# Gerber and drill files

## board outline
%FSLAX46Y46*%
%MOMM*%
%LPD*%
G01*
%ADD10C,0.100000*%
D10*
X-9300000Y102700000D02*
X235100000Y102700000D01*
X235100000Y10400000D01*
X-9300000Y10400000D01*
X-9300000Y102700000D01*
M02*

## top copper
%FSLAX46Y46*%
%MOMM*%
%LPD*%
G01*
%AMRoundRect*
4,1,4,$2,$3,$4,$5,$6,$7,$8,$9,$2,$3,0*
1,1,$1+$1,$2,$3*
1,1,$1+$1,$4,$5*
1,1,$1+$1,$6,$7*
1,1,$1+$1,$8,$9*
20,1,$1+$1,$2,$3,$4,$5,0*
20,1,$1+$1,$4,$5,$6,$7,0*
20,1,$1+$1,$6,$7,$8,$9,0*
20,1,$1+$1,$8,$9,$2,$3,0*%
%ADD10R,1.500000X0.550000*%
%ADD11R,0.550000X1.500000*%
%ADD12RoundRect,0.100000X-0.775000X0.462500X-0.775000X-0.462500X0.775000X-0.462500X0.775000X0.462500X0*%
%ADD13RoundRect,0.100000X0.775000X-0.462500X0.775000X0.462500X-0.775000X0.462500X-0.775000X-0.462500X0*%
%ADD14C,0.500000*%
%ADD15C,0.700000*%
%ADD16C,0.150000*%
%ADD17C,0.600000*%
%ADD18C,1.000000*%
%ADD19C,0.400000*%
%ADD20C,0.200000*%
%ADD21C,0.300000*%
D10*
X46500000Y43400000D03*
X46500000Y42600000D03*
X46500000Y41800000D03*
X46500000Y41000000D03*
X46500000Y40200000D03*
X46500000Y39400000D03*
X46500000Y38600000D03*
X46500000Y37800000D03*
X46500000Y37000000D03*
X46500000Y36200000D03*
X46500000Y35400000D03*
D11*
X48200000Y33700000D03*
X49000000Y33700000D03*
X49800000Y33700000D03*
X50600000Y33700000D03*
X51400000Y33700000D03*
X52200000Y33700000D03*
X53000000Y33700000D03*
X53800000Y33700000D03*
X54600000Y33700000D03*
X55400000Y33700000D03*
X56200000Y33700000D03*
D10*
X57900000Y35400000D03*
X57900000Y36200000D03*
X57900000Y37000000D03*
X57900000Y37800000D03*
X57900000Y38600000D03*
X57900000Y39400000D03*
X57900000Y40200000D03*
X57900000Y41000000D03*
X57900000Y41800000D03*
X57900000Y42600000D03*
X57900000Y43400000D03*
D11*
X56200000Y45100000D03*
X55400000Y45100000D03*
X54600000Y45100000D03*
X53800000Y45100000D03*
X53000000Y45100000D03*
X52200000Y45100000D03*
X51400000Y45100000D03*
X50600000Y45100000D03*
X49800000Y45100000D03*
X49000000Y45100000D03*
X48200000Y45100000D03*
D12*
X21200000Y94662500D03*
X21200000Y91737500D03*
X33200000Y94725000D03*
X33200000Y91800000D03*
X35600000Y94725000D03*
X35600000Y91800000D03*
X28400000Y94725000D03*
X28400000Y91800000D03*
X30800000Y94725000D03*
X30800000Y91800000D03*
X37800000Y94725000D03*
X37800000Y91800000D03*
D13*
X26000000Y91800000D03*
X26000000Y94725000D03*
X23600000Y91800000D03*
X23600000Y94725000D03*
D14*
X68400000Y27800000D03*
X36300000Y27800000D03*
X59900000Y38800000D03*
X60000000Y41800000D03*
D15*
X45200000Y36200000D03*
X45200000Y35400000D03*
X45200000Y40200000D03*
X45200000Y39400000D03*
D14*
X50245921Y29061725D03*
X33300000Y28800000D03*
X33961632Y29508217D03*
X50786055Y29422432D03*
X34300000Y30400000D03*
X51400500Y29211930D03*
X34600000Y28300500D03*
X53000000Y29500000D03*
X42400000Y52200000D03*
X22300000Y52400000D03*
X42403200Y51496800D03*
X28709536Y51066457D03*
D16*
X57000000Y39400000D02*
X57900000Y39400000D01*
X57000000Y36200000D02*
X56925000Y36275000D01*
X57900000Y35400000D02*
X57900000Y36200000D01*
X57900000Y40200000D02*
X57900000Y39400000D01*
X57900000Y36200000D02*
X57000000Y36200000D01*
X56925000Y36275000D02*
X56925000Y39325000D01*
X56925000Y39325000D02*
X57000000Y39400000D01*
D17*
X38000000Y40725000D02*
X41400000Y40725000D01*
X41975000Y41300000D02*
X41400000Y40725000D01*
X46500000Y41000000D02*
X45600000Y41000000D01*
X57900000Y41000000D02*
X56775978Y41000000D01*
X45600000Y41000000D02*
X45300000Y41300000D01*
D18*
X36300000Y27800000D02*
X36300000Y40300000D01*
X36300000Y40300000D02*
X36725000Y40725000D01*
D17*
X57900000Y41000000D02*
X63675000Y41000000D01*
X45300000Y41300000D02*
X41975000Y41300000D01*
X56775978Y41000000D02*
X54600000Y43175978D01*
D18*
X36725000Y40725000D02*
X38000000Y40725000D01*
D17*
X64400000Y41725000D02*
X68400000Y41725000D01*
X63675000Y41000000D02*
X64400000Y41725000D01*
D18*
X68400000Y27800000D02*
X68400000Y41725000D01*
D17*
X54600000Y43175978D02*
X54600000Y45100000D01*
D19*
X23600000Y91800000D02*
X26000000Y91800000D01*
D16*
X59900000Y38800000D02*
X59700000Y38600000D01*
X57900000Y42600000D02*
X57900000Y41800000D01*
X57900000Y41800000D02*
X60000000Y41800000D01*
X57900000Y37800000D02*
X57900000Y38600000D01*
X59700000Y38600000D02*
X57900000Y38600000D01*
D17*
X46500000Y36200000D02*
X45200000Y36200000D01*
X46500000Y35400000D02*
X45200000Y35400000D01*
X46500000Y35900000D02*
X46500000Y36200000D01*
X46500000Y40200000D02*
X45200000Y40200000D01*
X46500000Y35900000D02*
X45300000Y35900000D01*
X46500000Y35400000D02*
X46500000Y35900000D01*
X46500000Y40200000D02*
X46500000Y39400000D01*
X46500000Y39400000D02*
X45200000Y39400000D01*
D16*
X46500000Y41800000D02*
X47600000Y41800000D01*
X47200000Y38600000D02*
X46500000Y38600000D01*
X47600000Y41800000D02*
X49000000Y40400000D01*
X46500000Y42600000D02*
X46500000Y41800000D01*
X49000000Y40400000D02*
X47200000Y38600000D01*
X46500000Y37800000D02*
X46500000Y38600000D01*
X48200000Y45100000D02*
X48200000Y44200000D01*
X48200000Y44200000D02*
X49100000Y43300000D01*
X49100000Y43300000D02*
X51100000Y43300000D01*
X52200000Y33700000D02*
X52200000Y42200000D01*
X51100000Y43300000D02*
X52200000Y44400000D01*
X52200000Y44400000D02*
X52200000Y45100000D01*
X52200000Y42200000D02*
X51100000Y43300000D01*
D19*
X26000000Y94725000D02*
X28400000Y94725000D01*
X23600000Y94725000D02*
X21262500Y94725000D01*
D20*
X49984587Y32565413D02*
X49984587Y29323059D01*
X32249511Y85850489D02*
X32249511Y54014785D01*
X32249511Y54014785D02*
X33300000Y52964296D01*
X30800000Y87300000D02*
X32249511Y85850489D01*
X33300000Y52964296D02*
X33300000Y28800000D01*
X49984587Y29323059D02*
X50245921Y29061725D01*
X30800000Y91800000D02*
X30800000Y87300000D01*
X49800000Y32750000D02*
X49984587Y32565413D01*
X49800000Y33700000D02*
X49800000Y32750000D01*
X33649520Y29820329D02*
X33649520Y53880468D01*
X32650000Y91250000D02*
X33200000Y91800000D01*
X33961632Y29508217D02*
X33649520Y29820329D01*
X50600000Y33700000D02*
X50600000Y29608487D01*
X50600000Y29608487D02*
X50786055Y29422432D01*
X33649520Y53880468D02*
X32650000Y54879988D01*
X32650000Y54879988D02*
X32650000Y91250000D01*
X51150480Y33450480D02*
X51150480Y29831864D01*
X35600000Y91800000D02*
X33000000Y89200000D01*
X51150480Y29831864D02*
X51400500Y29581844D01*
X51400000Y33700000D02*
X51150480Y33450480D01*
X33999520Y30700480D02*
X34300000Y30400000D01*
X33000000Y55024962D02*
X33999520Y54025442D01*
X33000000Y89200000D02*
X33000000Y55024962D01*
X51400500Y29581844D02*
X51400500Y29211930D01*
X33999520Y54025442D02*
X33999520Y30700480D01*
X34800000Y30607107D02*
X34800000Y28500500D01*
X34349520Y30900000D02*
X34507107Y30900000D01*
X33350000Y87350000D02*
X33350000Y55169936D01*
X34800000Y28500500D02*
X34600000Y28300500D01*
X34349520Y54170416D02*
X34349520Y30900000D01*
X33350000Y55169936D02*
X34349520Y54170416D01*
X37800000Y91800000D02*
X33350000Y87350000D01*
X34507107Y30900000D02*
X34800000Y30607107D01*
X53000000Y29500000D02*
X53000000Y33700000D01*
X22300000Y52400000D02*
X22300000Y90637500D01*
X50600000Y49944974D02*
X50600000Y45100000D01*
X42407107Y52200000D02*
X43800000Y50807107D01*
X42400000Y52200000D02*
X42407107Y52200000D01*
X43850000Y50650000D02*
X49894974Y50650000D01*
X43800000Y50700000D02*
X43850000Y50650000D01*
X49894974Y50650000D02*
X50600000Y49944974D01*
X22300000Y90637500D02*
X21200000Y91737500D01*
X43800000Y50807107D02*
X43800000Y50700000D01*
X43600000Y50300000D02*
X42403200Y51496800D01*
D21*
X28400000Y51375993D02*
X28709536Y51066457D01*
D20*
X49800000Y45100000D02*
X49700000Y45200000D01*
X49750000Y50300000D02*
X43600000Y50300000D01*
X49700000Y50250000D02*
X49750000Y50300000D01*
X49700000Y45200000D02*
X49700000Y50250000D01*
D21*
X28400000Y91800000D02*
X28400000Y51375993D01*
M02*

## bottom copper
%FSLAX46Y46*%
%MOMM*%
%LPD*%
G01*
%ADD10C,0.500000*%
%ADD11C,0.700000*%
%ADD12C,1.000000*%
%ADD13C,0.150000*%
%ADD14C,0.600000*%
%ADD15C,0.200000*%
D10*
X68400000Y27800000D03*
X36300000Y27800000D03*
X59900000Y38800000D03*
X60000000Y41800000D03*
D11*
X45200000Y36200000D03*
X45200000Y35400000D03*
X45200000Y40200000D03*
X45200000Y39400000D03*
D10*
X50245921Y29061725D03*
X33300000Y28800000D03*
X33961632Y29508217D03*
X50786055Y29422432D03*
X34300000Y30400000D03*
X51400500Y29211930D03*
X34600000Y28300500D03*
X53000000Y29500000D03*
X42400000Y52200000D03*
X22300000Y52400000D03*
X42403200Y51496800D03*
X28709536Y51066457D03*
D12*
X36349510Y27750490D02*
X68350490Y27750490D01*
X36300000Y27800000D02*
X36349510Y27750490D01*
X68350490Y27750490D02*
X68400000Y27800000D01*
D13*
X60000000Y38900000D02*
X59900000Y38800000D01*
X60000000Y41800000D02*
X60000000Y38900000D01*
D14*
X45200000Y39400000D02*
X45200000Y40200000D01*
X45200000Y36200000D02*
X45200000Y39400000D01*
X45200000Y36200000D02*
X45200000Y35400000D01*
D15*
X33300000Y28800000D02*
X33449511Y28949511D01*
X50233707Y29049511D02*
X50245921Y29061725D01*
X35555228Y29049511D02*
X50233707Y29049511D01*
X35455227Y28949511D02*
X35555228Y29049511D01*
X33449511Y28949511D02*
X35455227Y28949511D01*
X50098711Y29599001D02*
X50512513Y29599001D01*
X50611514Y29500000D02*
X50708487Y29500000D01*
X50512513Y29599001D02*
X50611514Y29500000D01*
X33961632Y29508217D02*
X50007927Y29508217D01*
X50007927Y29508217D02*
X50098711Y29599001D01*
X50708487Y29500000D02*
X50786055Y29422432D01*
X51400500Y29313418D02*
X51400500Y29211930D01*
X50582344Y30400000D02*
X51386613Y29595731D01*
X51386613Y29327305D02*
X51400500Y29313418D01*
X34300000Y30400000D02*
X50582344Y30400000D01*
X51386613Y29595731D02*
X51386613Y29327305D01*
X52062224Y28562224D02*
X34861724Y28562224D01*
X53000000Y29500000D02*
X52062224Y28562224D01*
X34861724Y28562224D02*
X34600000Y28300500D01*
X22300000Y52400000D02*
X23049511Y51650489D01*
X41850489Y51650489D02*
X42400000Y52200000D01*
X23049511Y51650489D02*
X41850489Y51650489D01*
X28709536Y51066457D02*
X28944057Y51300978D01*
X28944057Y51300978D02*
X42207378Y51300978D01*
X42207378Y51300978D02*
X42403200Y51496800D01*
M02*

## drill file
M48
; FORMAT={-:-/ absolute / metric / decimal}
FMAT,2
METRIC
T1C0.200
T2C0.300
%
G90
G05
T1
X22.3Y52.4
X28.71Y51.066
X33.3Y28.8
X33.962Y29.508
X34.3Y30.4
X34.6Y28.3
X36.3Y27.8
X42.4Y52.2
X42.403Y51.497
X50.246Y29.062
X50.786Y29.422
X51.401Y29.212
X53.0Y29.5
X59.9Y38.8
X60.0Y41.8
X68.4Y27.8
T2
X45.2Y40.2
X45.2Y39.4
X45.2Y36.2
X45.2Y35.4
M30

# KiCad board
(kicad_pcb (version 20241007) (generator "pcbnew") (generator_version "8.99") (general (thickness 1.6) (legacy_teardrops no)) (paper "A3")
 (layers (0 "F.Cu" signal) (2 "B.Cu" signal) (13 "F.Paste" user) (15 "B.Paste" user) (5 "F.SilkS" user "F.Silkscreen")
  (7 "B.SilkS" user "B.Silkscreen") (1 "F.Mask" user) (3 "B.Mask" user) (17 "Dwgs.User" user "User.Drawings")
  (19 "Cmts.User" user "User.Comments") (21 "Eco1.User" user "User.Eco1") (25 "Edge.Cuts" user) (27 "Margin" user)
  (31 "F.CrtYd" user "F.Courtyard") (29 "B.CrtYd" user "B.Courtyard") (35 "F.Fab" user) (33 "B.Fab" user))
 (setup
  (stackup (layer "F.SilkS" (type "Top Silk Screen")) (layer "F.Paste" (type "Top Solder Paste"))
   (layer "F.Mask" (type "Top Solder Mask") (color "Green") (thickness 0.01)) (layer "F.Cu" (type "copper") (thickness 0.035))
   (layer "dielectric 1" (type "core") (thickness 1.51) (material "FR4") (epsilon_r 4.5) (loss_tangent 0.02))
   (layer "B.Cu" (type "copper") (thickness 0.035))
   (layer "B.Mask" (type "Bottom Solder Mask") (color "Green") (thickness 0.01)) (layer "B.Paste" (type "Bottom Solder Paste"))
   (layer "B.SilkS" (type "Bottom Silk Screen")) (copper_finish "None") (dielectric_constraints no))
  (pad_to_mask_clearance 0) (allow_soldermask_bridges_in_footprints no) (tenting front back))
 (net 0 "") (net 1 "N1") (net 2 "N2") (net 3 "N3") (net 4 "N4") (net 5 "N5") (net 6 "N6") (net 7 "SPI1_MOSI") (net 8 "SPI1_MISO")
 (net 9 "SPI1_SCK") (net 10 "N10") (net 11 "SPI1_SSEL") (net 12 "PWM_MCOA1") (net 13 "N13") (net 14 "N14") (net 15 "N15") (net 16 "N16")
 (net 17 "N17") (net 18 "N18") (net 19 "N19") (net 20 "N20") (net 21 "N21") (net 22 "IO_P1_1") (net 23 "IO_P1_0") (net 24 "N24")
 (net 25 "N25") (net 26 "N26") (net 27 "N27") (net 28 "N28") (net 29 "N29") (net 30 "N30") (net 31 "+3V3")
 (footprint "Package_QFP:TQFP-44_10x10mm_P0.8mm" (layer "F.Cu") (at 52.2 -39.4)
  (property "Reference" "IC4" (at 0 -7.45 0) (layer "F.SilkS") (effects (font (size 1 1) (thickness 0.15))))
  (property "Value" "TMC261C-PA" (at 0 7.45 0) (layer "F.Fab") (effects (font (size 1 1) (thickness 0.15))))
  (pad "1" smd rect (at -5.7 -4) (size 1.5 0.55) (layers "F.Cu" "F.Mask" "F.Paste"))
  (pad "2" smd rect (at -5.7 -3.2) (size 1.5 0.55) (layers "F.Cu" "F.Mask" "F.Paste") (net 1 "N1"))
  (pad "3" smd rect (at -5.7 -2.4) (size 1.5 0.55) (layers "F.Cu" "F.Mask" "F.Paste") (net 1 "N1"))
  (pad "4" smd rect (at -5.7 -1.6) (size 1.5 0.55) (layers "F.Cu" "F.Mask" "F.Paste") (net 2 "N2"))
  (pad "5" smd rect (at -5.7 -0.8) (size 1.5 0.55) (layers "F.Cu" "F.Mask" "F.Paste") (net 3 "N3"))
  (pad "6" smd rect (at -5.7 0) (size 1.5 0.55) (layers "F.Cu" "F.Mask" "F.Paste") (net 3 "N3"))
  (pad "7" smd rect (at -5.7 0.8) (size 1.5 0.55) (layers "F.Cu" "F.Mask" "F.Paste") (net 1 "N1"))
  (pad "8" smd rect (at -5.7 1.6) (size 1.5 0.55) (layers "F.Cu" "F.Mask" "F.Paste") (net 1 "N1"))
  (pad "9" smd rect (at -5.7 2.4) (size 1.5 0.55) (layers "F.Cu" "F.Mask" "F.Paste") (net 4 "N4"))
  (pad "10" smd rect (at -5.7 3.2) (size 1.5 0.55) (layers "F.Cu" "F.Mask" "F.Paste") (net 3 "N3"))
  (pad "11" smd rect (at -5.7 4) (size 1.5 0.55) (layers "F.Cu" "F.Mask" "F.Paste") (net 3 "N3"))
  (pad "12" smd rect (at -4 5.7 90) (size 1.5 0.55) (layers "F.Cu" "F.Mask" "F.Paste") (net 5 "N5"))
  (pad "13" smd rect (at -3.2 5.7 90) (size 1.5 0.55) (layers "F.Cu" "F.Mask" "F.Paste") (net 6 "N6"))
  (pad "14" smd rect (at -2.4 5.7 90) (size 1.5 0.55) (layers "F.Cu" "F.Mask" "F.Paste") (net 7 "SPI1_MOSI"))
  (pad "15" smd rect (at -1.6 5.7 90) (size 1.5 0.55) (layers "F.Cu" "F.Mask" "F.Paste") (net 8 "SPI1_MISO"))
  (pad "16" smd rect (at -0.8 5.7 90) (size 1.5 0.55) (layers "F.Cu" "F.Mask" "F.Paste") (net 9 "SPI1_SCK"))
  (pad "17" smd rect (at 0 5.7 90) (size 1.5 0.55) (layers "F.Cu" "F.Mask" "F.Paste") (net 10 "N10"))
  (pad "18" smd rect (at 0.8 5.7 90) (size 1.5 0.55) (layers "F.Cu" "F.Mask" "F.Paste") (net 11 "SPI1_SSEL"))
  (pad "19" smd rect (at 1.6 5.7 90) (size 1.5 0.55) (layers "F.Cu" "F.Mask" "F.Paste") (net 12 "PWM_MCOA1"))
  (pad "20" smd rect (at 2.4 5.7 90) (size 1.5 0.55) (layers "F.Cu" "F.Mask" "F.Paste"))
  (pad "21" smd rect (at 3.2 5.7 90) (size 1.5 0.55) (layers "F.Cu" "F.Mask" "F.Paste") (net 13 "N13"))
  (pad "22" smd rect (at 4 5.7 90) (size 1.5 0.55) (layers "F.Cu" "F.Mask" "F.Paste") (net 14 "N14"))
  (pad "23" smd rect (at 5.7 4) (size 1.5 0.55) (layers "F.Cu" "F.Mask" "F.Paste") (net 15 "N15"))
  (pad "24" smd rect (at 5.7 3.2) (size 1.5 0.55) (layers "F.Cu" "F.Mask" "F.Paste") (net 15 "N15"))
  (pad "25" smd rect (at 5.7 2.4) (size 1.5 0.55) (layers "F.Cu" "F.Mask" "F.Paste") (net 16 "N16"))
  (pad "26" smd rect (at 5.7 1.6) (size 1.5 0.55) (layers "F.Cu" "F.Mask" "F.Paste") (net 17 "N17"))
  (pad "27" smd rect (at 5.7 0.8) (size 1.5 0.55) (layers "F.Cu" "F.Mask" "F.Paste") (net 17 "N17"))
  (pad "28" smd rect (at 5.7 0) (size 1.5 0.55) (layers "F.Cu" "F.Mask" "F.Paste") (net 15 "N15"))
  (pad "29" smd rect (at 5.7 -0.8) (size 1.5 0.55) (layers "F.Cu" "F.Mask" "F.Paste") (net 15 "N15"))
  (pad "30" smd rect (at 5.7 -1.6) (size 1.5 0.55) (layers "F.Cu" "F.Mask" "F.Paste") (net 2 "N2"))
  (pad "31" smd rect (at 5.7 -2.4) (size 1.5 0.55) (layers "F.Cu" "F.Mask" "F.Paste") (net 17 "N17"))
  (pad "32" smd rect (at 5.7 -3.2) (size 1.5 0.55) (layers "F.Cu" "F.Mask" "F.Paste") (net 17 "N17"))
  (pad "33" smd rect (at 5.7 -4) (size 1.5 0.55) (layers "F.Cu" "F.Mask" "F.Paste"))
  (pad "34" smd rect (at 4 -5.7 90) (size 1.5 0.55) (layers "F.Cu" "F.Mask" "F.Paste"))
  (pad "35" smd rect (at 3.2 -5.7 90) (size 1.5 0.55) (layers "F.Cu" "F.Mask" "F.Paste") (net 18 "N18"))
  (pad "36" smd rect (at 2.4 -5.7 90) (size 1.5 0.55) (layers "F.Cu" "F.Mask" "F.Paste") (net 2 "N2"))
  (pad "37" smd rect (at 1.6 -5.7 90) (size 1.5 0.55) (layers "F.Cu" "F.Mask" "F.Paste") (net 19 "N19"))
  (pad "38" smd rect (at 0.8 -5.7 90) (size 1.5 0.55) (layers "F.Cu" "F.Mask" "F.Paste") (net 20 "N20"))
  (pad "39" smd rect (at 0 -5.7 90) (size 1.5 0.55) (layers "F.Cu" "F.Mask" "F.Paste") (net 10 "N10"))
  (pad "40" smd rect (at -0.8 -5.7 90) (size 1.5 0.55) (layers "F.Cu" "F.Mask" "F.Paste") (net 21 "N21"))
  (pad "41" smd rect (at -1.6 -5.7 90) (size 1.5 0.55) (layers "F.Cu" "F.Mask" "F.Paste") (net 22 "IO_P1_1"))
  (pad "42" smd rect (at -2.4 -5.7 90) (size 1.5 0.55) (layers "F.Cu" "F.Mask" "F.Paste") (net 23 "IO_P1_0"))
  (pad "43" smd rect (at -3.2 -5.7 90) (size 1.5 0.55) (layers "F.Cu" "F.Mask" "F.Paste") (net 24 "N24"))
  (pad "44" smd rect (at -4 -5.7 90) (size 1.5 0.55) (layers "F.Cu" "F.Mask" "F.Paste") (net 10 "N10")))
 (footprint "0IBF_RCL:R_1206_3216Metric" (layer "F.Cu") (at 21.2 -93.2 -90)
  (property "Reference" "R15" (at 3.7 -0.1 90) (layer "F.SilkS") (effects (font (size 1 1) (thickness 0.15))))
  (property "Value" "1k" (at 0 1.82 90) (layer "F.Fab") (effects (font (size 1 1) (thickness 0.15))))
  (pad "1" smd roundrect (at -1.4625 0 270) (size 1.125 1.75) (layers "F.Cu" "F.Mask" "F.Paste") (roundrect_rratio 0.08888888889)
   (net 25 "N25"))
  (pad "2" smd roundrect (at 1.4625 0 270) (size 1.125 1.75) (layers "F.Cu" "F.Mask" "F.Paste") (roundrect_rratio 0.08888888889)
   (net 22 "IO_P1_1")))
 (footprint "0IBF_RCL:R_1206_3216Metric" (layer "F.Cu") (at 33.2 -93.2625 -90)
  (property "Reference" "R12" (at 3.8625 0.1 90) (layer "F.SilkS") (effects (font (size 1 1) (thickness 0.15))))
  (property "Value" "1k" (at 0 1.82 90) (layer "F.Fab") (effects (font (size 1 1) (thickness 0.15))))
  (pad "1" smd roundrect (at -1.4625 0 270) (size 1.125 1.75) (layers "F.Cu" "F.Mask" "F.Paste") (roundrect_rratio 0.08888888889)
   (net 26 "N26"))
  (pad "2" smd roundrect (at 1.4625 0 270) (size 1.125 1.75) (layers "F.Cu" "F.Mask" "F.Paste") (roundrect_rratio 0.08888888889)
   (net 8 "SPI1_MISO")))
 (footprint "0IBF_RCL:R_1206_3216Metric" (layer "F.Cu") (at 35.6 -93.2625 -90)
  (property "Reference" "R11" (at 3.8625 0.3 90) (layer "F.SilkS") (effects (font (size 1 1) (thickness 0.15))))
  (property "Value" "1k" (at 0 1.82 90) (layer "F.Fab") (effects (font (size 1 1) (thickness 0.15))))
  (pad "1" smd roundrect (at -1.4625 0 270) (size 1.125 1.75) (layers "F.Cu" "F.Mask" "F.Paste") (roundrect_rratio 0.08888888889)
   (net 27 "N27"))
  (pad "2" smd roundrect (at 1.4625 0 270) (size 1.125 1.75) (layers "F.Cu" "F.Mask" "F.Paste") (roundrect_rratio 0.08888888889)
   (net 9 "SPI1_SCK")))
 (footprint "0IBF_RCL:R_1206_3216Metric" (layer "F.Cu") (at 28.4 -93.2625 -90)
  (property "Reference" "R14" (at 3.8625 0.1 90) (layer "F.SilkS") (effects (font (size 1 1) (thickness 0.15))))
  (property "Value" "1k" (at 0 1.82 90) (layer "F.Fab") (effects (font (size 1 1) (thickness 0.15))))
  (pad "1" smd roundrect (at -1.4625 0 270) (size 1.125 1.75) (layers "F.Cu" "F.Mask" "F.Paste") (roundrect_rratio 0.08888888889)
   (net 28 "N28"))
  (pad "2" smd roundrect (at 1.4625 0 270) (size 1.125 1.75) (layers "F.Cu" "F.Mask" "F.Paste") (roundrect_rratio 0.08888888889)
   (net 23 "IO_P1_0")))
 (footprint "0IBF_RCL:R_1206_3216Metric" (layer "F.Cu") (at 30.8 -93.2625 -90)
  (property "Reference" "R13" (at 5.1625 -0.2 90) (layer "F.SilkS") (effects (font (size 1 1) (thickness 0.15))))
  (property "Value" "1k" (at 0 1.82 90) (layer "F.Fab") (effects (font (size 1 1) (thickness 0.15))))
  (pad "1" smd roundrect (at -1.4625 0 270) (size 1.125 1.75) (layers "F.Cu" "F.Mask" "F.Paste") (roundrect_rratio 0.08888888889)
   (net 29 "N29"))
  (pad "2" smd roundrect (at 1.4625 0 270) (size 1.125 1.75) (layers "F.Cu" "F.Mask" "F.Paste") (roundrect_rratio 0.08888888889)
   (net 7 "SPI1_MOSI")))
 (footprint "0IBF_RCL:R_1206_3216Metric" (layer "F.Cu") (at 37.8 -93.2625 -90)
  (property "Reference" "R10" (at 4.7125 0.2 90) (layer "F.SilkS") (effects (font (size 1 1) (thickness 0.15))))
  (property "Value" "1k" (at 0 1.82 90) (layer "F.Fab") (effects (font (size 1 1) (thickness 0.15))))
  (pad "1" smd roundrect (at -1.4625 0 270) (size 1.125 1.75) (layers "F.Cu" "F.Mask" "F.Paste") (roundrect_rratio 0.08888888889)
   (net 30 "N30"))
  (pad "2" smd roundrect (at 1.4625 0 270) (size 1.125 1.75) (layers "F.Cu" "F.Mask" "F.Paste") (roundrect_rratio 0.08888888889)
   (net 11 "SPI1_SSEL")))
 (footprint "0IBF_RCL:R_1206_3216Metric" (layer "F.Cu") (at 26 -93.2625 90)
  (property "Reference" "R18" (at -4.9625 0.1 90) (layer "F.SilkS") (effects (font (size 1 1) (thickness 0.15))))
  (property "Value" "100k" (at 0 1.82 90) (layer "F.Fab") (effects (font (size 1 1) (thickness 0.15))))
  (pad "1" smd roundrect (at -1.4625 0 90) (size 1.125 1.75) (layers "F.Cu" "F.Mask" "F.Paste") (roundrect_rratio 0.08888888889)
   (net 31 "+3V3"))
  (pad "2" smd roundrect (at 1.4625 0 90) (size 1.125 1.75) (layers "F.Cu" "F.Mask" "F.Paste") (roundrect_rratio 0.08888888889)
   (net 28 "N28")))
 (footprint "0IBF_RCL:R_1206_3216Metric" (layer "F.Cu") (at 23.6 -93.2625 90)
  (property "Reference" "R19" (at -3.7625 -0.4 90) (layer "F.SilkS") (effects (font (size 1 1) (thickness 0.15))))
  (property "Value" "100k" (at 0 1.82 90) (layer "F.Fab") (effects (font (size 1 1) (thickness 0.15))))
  (pad "1" smd roundrect (at -1.4625 0 90) (size 1.125 1.75) (layers "F.Cu" "F.Mask" "F.Paste") (roundrect_rratio 0.08888888889)
   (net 31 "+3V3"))
  (pad "2" smd roundrect (at 1.4625 0 90) (size 1.125 1.75) (layers "F.Cu" "F.Mask" "F.Paste") (roundrect_rratio 0.08888888889)
   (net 25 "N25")))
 (gr_rect (start -9.3 -102.7) (end 235.1 -10.4) (stroke (width 0.1) (type default)) (fill none) (layer "Edge.Cuts"))
 (segment (start 57 -39.4) (end 57.9 -39.4) (width 0.15) (layer "F.Cu") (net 15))
 (segment (start 57 -36.2) (end 56.925 -36.275) (width 0.15) (layer "F.Cu") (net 15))
 (segment (start 57.9 -35.4) (end 57.9 -36.2) (width 0.15) (layer "F.Cu") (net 15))
 (segment (start 57.9 -40.2) (end 57.9 -39.4) (width 0.15) (layer "F.Cu") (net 15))
 (segment (start 57.9 -36.2) (end 57 -36.2) (width 0.15) (layer "F.Cu") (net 15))
 (segment (start 56.925 -36.275) (end 56.925 -39.325) (width 0.15) (layer "F.Cu") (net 15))
 (segment (start 56.925 -39.325) (end 57 -39.4) (width 0.15) (layer "F.Cu") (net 15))
 (segment (start 38 -40.725) (end 41.4 -40.725) (width 0.6) (layer "F.Cu") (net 2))
 (segment (start 41.975 -41.3) (end 41.4 -40.725) (width 0.6) (layer "F.Cu") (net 2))
 (segment (start 46.5 -41) (end 45.6 -41) (width 0.6) (layer "F.Cu") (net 2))
 (segment (start 57.9 -41) (end 56.775978 -41) (width 0.6) (layer "F.Cu") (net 2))
 (segment (start 45.6 -41) (end 45.3 -41.3) (width 0.6) (layer "F.Cu") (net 2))
 (segment (start 36.3 -27.8) (end 36.3 -40.3) (width 1) (layer "F.Cu") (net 2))
 (segment (start 36.3 -40.3) (end 36.725 -40.725) (width 1) (layer "F.Cu") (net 2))
 (segment (start 57.9 -41) (end 63.675 -41) (width 0.6) (layer "F.Cu") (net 2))
 (segment (start 45.3 -41.3) (end 41.975 -41.3) (width 0.6) (layer "F.Cu") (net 2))
 (segment (start 56.775978 -41) (end 54.6 -43.175978) (width 0.6) (layer "F.Cu") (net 2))
 (segment (start 36.725 -40.725) (end 38 -40.725) (width 1) (layer "F.Cu") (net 2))
 (segment (start 64.4 -41.725) (end 68.4 -41.725) (width 0.6) (layer "F.Cu") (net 2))
 (segment (start 63.675 -41) (end 64.4 -41.725) (width 0.6) (layer "F.Cu") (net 2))
 (segment (start 68.4 -27.8) (end 68.4 -41.725) (width 1) (layer "F.Cu") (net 2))
 (segment (start 54.6 -43.175978) (end 54.6 -45.1) (width 0.6) (layer "F.Cu") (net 2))
 (via (at 68.4 -27.8) (size 0.5) (drill 0.2) (layers "F.Cu" "B.Cu") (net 2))
 (via (at 36.3 -27.8) (size 0.5) (drill 0.2) (layers "F.Cu" "B.Cu") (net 2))
 (segment (start 36.34951 -27.75049) (end 68.35049 -27.75049) (width 1) (layer "B.Cu") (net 2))
 (segment (start 36.3 -27.8) (end 36.34951 -27.75049) (width 1) (layer "B.Cu") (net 2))
 (segment (start 68.35049 -27.75049) (end 68.4 -27.8) (width 1) (layer "B.Cu") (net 2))
 (segment (start 23.6 -91.8) (end 26 -91.8) (width 0.4) (layer "F.Cu") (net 31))
 (segment (start 59.9 -38.8) (end 59.7 -38.6) (width 0.15) (layer "F.Cu") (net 17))
 (segment (start 57.9 -42.6) (end 57.9 -41.8) (width 0.15) (layer "F.Cu") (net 17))
 (segment (start 57.9 -41.8) (end 60 -41.8) (width 0.15) (layer "F.Cu") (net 17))
 (segment (start 57.9 -37.8) (end 57.9 -38.6) (width 0.15) (layer "F.Cu") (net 17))
 (segment (start 59.7 -38.6) (end 57.9 -38.6) (width 0.15) (layer "F.Cu") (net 17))
 (via (at 59.9 -38.8) (size 0.5) (drill 0.2) (layers "F.Cu" "B.Cu") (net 17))
 (via (at 60 -41.8) (size 0.5) (drill 0.2) (layers "F.Cu" "B.Cu") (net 17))
 (segment (start 60 -38.9) (end 59.9 -38.8) (width 0.15) (layer "B.Cu") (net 17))
 (segment (start 60 -41.8) (end 60 -38.9) (width 0.15) (layer "B.Cu") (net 17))
 (segment (start 46.5 -36.2) (end 45.2 -36.2) (width 0.6) (layer "F.Cu") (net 3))
 (segment (start 46.5 -35.4) (end 45.2 -35.4) (width 0.6) (layer "F.Cu") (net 3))
 (segment (start 46.5 -35.9) (end 46.5 -36.2) (width 0.6) (layer "F.Cu") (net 3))
 (segment (start 46.5 -40.2) (end 45.2 -40.2) (width 0.6) (layer "F.Cu") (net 3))
 (segment (start 46.5 -35.9) (end 45.3 -35.9) (width 0.6) (layer "F.Cu") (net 3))
 (segment (start 46.5 -35.4) (end 46.5 -35.9) (width 0.6) (layer "F.Cu") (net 3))
 (segment (start 46.5 -40.2) (end 46.5 -39.4) (width 0.6) (layer "F.Cu") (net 3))
 (segment (start 46.5 -39.4) (end 45.2 -39.4) (width 0.6) (layer "F.Cu") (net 3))
 (via (at 45.2 -36.2) (size 0.7) (drill 0.3) (layers "F.Cu" "B.Cu") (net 3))
 (via (at 45.2 -35.4) (size 0.7) (drill 0.3) (layers "F.Cu" "B.Cu") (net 3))
 (via (at 45.2 -40.2) (size 0.7) (drill 0.3) (layers "F.Cu" "B.Cu") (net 3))
 (via (at 45.2 -39.4) (size 0.7) (drill 0.3) (layers "F.Cu" "B.Cu") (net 3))
 (segment (start 45.2 -39.4) (end 45.2 -40.2) (width 0.6) (layer "B.Cu") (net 3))
 (segment (start 45.2 -36.2) (end 45.2 -39.4) (width 0.6) (layer "B.Cu") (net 3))
 (segment (start 45.2 -36.2) (end 45.2 -35.4) (width 0.6) (layer "B.Cu") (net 3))
 (segment (start 46.5 -41.8) (end 47.6 -41.8) (width 0.15) (layer "F.Cu") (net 1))
 (segment (start 47.2 -38.6) (end 46.5 -38.6) (width 0.15) (layer "F.Cu") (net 1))
 (segment (start 47.6 -41.8) (end 49 -40.4) (width 0.15) (layer "F.Cu") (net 1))
 (segment (start 46.5 -42.6) (end 46.5 -41.8) (width 0.15) (layer "F.Cu") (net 1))
 (segment (start 49 -40.4) (end 47.2 -38.6) (width 0.15) (layer "F.Cu") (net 1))
 (segment (start 46.5 -37.8) (end 46.5 -38.6) (width 0.15) (layer "F.Cu") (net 1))
 (segment (start 48.2 -45.1) (end 48.2 -44.2) (width 0.15) (layer "F.Cu") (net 10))
 (segment (start 48.2 -44.2) (end 49.1 -43.3) (width 0.15) (layer "F.Cu") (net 10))
 (segment (start 49.1 -43.3) (end 51.1 -43.3) (width 0.15) (layer "F.Cu") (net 10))
 (segment (start 52.2 -33.7) (end 52.2 -42.2) (width 0.15) (layer "F.Cu") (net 10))
 (segment (start 51.1 -43.3) (end 52.2 -44.4) (width 0.15) (layer "F.Cu") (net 10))
 (segment (start 52.2 -44.4) (end 52.2 -45.1) (width 0.15) (layer "F.Cu") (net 10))
 (segment (start 52.2 -42.2) (end 51.1 -43.3) (width 0.15) (layer "F.Cu") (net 10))
 (segment (start 26 -94.725) (end 28.4 -94.725) (width 0.4) (layer "F.Cu") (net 28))
 (segment (start 23.6 -94.725) (end 21.2625 -94.725) (width 0.4) (layer "F.Cu") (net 25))
 (segment (start 49.984587 -32.565413) (end 49.984587 -29.323059) (width 0.2) (layer "F.Cu") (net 7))
 (segment (start 32.249511 -85.850489) (end 32.249511 -54.014785) (width 0.2) (layers "F.Cu" "F.Mask") (solder_mask_margin 1) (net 7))
 (segment (start 32.249511 -54.014785) (end 33.3 -52.964296) (width 0.2) (layer "F.Cu") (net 7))
 (segment (start 30.8 -87.3) (end 32.249511 -85.850489) (width 0.2) (layer "F.Cu") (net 7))
 (segment (start 33.3 -52.964296) (end 33.3 -28.8) (width 0.2) (layer "F.Cu") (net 7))
 (segment (start 49.984587 -29.323059) (end 50.245921 -29.061725) (width 0.2) (layer "F.Cu") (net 7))
 (segment (start 30.8 -91.8) (end 30.8 -87.3) (width 0.2) (layer "F.Cu") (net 7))
 (segment (start 49.8 -32.75) (end 49.984587 -32.565413) (width 0.2) (layer "F.Cu") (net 7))
 (segment (start 49.8 -33.7) (end 49.8 -32.75) (width 0.2) (layer "F.Cu") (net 7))
 (via (at 50.245921 -29.061725) (size 0.5) (drill 0.2) (layers "F.Cu" "B.Cu") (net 7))
 (via (at 33.3 -28.8) (size 0.5) (drill 0.2) (layers "F.Cu" "B.Cu") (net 7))
 (segment (start 33.3 -28.8) (end 33.449511 -28.949511) (width 0.2) (layer "B.Cu") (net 7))
 (segment (start 50.233707 -29.049511) (end 50.245921 -29.061725) (width 0.2) (layer "B.Cu") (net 7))
 (segment (start 35.555228 -29.049511) (end 50.233707 -29.049511) (width 0.2) (layer "B.Cu") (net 7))
 (segment (start 35.455227 -28.949511) (end 35.555228 -29.049511) (width 0.2) (layer "B.Cu") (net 7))
 (segment (start 33.449511 -28.949511) (end 35.455227 -28.949511) (width 0.2) (layer "B.Cu") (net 7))
 (segment (start 33.64952 -29.820329) (end 33.64952 -53.880468) (width 0.2) (layer "F.Cu") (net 8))
 (segment (start 32.65 -91.25) (end 33.2 -91.8) (width 0.2) (layer "F.Cu") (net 8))
 (segment (start 33.961632 -29.508217) (end 33.64952 -29.820329) (width 0.2) (layer "F.Cu") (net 8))
 (segment (start 50.6 -33.7) (end 50.6 -29.608487) (width 0.2) (layer "F.Cu") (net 8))
 (segment (start 50.6 -29.608487) (end 50.786055 -29.422432) (width 0.2) (layer "F.Cu") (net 8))
 (segment (start 33.64952 -53.880468) (end 32.65 -54.879988) (width 0.2) (layer "F.Cu") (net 8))
 (segment (start 32.65 -54.879988) (end 32.65 -91.25) (width 0.2) (layer "F.Cu") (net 8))
 (via (at 33.961632 -29.508217) (size 0.5) (drill 0.2) (layers "F.Cu" "B.Cu") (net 8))
 (via (at 50.786055 -29.422432) (size 0.5) (drill 0.2) (layers "F.Cu" "B.Cu") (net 8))
 (segment (start 50.098711 -29.599001) (end 50.512513 -29.599001) (width 0.2) (layer "B.Cu") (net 8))
 (segment (start 50.611514 -29.5) (end 50.708487 -29.5) (width 0.2) (layer "B.Cu") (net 8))
 (segment (start 50.512513 -29.599001) (end 50.611514 -29.5) (width 0.2) (layer "B.Cu") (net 8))
 (segment (start 33.961632 -29.508217) (end 50.007927 -29.508217) (width 0.2) (layer "B.Cu") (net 8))
 (segment (start 50.007927 -29.508217) (end 50.098711 -29.599001) (width 0.2) (layer "B.Cu") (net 8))
 (segment (start 50.708487 -29.5) (end 50.786055 -29.422432) (width 0.2) (layer "B.Cu") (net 8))
 (segment (start 51.15048 -33.45048) (end 51.15048 -29.831864) (width 0.2) (layer "F.Cu") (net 9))
 (segment (start 35.6 -91.8) (end 33 -89.2) (width 0.2) (layer "F.Cu") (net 9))
 (segment (start 51.15048 -29.831864) (end 51.4005 -29.581844) (width 0.2) (layer "F.Cu") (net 9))
 (segment (start 51.4 -33.7) (end 51.15048 -33.45048) (width 0.2) (layer "F.Cu") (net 9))
 (segment (start 33.99952 -30.70048) (end 34.3 -30.4) (width 0.2) (layer "F.Cu") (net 9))
 (segment (start 33 -55.024962) (end 33.99952 -54.025442) (width 0.2) (layer "F.Cu") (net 9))
 (segment (start 33 -89.2) (end 33 -55.024962) (width 0.2) (layer "F.Cu") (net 9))
 (segment (start 51.4005 -29.581844) (end 51.4005 -29.21193) (width 0.2) (layer "F.Cu") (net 9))
 (segment (start 33.99952 -54.025442) (end 33.99952 -30.70048) (width 0.2) (layer "F.Cu") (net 9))
 (via (at 34.3 -30.4) (size 0.5) (drill 0.2) (layers "F.Cu" "B.Cu") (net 9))
 (via (at 51.4005 -29.21193) (size 0.5) (drill 0.2) (layers "F.Cu" "B.Cu") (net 9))
 (segment (start 51.4005 -29.313418) (end 51.4005 -29.21193) (width 0.2) (layer "B.Cu") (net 9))
 (segment (start 50.582344 -30.4) (end 51.386613 -29.595731) (width 0.2) (layer "B.Cu") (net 9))
 (segment (start 51.386613 -29.327305) (end 51.4005 -29.313418) (width 0.2) (layer "B.Cu") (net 9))
 (segment (start 34.3 -30.4) (end 50.582344 -30.4) (width 0.2) (layer "B.Cu") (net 9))
 (segment (start 51.386613 -29.595731) (end 51.386613 -29.327305) (width 0.2) (layer "B.Cu") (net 9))
 (segment (start 34.8 -30.607107) (end 34.8 -28.5005) (width 0.2) (layer "F.Cu") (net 11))
 (segment (start 34.34952 -30.9) (end 34.507107 -30.9) (width 0.2) (layer "F.Cu") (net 11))
 (segment (start 33.35 -87.35) (end 33.35 -55.169936) (width 0.2) (layer "F.Cu") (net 11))
 (segment (start 34.8 -28.5005) (end 34.6 -28.3005) (width 0.2) (layer "F.Cu") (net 11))
 (segment (start 34.34952 -54.170416) (end 34.34952 -30.9) (width 0.2) (layer "F.Cu") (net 11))
 (segment (start 33.35 -55.169936) (end 34.34952 -54.170416) (width 0.2) (layer "F.Cu") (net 11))
 (segment (start 37.8 -91.8) (end 33.35 -87.35) (width 0.2) (layer "F.Cu") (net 11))
 (segment (start 34.507107 -30.9) (end 34.8 -30.607107) (width 0.2) (layer "F.Cu") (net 11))
 (segment (start 53 -29.5) (end 53 -33.7) (width 0.2) (layer "F.Cu") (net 11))
 (via (at 34.6 -28.3005) (size 0.5) (drill 0.2) (layers "F.Cu" "B.Cu") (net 11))
 (via (at 53 -29.5) (size 0.5) (drill 0.2) (layers "F.Cu" "B.Cu") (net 11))
 (segment (start 52.062224 -28.562224) (end 34.861724 -28.562224) (width 0.2) (layer "B.Cu") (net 11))
 (segment (start 53 -29.5) (end 52.062224 -28.562224) (width 0.2) (layer "B.Cu") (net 11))
 (segment (start 34.861724 -28.562224) (end 34.6 -28.3005) (width 0.2) (layer "B.Cu") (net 11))
 (segment (start 22.3 -52.4) (end 22.3 -90.6375) (width 0.2) (layer "F.Cu") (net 22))
 (segment (start 50.6 -49.944974) (end 50.6 -45.1) (width 0.2) (layer "F.Cu") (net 22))
 (segment (start 42.407107 -52.2) (end 43.8 -50.807107) (width 0.2) (layer "F.Cu") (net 22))
 (segment (start 42.4 -52.2) (end 42.407107 -52.2) (width 0.2) (layer "F.Cu") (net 22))
 (segment (start 43.85 -50.65) (end 49.894974 -50.65) (width 0.2) (layer "F.Cu") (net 22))
 (segment (start 43.8 -50.7) (end 43.85 -50.65) (width 0.2) (layer "F.Cu") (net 22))
 (segment (start 49.894974 -50.65) (end 50.6 -49.944974) (width 0.2) (layer "F.Cu") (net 22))
 (segment (start 22.3 -90.6375) (end 21.2 -91.7375) (width 0.2) (layer "F.Cu") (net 22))
 (segment (start 43.8 -50.807107) (end 43.8 -50.7) (width 0.2) (layer "F.Cu") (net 22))
 (via (at 42.4 -52.2) (size 0.5) (drill 0.2) (layers "F.Cu" "B.Cu") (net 22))
 (via (at 22.3 -52.4) (size 0.5) (drill 0.2) (layers "F.Cu" "B.Cu") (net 22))
 (segment (start 22.3 -52.4) (end 23.049511 -51.650489) (width 0.2) (layer "B.Cu") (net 22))
 (segment (start 41.850489 -51.650489) (end 42.4 -52.2) (width 0.2) (layer "B.Cu") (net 22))
 (segment (start 23.049511 -51.650489) (end 41.850489 -51.650489) (width 0.2) (layer "B.Cu") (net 22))
 (segment (start 43.6 -50.3) (end 42.4032 -51.4968) (width 0.2) (layer "F.Cu") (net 23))
 (segment (start 28.4 -51.375993) (end 28.709536 -51.066457) (width 0.3) (layer "F.Cu") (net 23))
 (segment (start 49.8 -45.1) (end 49.7 -45.2) (width 0.2) (layer "F.Cu") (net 23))
 (segment (start 49.75 -50.3) (end 43.6 -50.3) (width 0.2) (layer "F.Cu") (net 23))
 (segment (start 49.7 -50.25) (end 49.75 -50.3) (width 0.2) (layer "F.Cu") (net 23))
 (segment (start 49.7 -45.2) (end 49.7 -50.25) (width 0.2) (layer "F.Cu") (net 23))
 (segment (start 28.4 -91.8) (end 28.4 -51.375993) (width 0.3) (layer "F.Cu") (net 23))
 (via (at 42.4032 -51.4968) (size 0.5) (drill 0.2) (layers "F.Cu" "B.Cu") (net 23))
 (via (at 28.709536 -51.066457) (size 0.5) (drill 0.2) (layers "F.Cu" "B.Cu") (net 23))
 (segment (start 28.709536 -51.066457) (end 28.944057 -51.300978) (width 0.2) (layer "B.Cu") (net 23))
 (segment (start 28.944057 -51.300978) (end 42.207378 -51.300978) (width 0.2) (layer "B.Cu") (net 23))
 (segment (start 42.207378 -51.300978) (end 42.4032 -51.4968) (width 0.2) (layer "B.Cu") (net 23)))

